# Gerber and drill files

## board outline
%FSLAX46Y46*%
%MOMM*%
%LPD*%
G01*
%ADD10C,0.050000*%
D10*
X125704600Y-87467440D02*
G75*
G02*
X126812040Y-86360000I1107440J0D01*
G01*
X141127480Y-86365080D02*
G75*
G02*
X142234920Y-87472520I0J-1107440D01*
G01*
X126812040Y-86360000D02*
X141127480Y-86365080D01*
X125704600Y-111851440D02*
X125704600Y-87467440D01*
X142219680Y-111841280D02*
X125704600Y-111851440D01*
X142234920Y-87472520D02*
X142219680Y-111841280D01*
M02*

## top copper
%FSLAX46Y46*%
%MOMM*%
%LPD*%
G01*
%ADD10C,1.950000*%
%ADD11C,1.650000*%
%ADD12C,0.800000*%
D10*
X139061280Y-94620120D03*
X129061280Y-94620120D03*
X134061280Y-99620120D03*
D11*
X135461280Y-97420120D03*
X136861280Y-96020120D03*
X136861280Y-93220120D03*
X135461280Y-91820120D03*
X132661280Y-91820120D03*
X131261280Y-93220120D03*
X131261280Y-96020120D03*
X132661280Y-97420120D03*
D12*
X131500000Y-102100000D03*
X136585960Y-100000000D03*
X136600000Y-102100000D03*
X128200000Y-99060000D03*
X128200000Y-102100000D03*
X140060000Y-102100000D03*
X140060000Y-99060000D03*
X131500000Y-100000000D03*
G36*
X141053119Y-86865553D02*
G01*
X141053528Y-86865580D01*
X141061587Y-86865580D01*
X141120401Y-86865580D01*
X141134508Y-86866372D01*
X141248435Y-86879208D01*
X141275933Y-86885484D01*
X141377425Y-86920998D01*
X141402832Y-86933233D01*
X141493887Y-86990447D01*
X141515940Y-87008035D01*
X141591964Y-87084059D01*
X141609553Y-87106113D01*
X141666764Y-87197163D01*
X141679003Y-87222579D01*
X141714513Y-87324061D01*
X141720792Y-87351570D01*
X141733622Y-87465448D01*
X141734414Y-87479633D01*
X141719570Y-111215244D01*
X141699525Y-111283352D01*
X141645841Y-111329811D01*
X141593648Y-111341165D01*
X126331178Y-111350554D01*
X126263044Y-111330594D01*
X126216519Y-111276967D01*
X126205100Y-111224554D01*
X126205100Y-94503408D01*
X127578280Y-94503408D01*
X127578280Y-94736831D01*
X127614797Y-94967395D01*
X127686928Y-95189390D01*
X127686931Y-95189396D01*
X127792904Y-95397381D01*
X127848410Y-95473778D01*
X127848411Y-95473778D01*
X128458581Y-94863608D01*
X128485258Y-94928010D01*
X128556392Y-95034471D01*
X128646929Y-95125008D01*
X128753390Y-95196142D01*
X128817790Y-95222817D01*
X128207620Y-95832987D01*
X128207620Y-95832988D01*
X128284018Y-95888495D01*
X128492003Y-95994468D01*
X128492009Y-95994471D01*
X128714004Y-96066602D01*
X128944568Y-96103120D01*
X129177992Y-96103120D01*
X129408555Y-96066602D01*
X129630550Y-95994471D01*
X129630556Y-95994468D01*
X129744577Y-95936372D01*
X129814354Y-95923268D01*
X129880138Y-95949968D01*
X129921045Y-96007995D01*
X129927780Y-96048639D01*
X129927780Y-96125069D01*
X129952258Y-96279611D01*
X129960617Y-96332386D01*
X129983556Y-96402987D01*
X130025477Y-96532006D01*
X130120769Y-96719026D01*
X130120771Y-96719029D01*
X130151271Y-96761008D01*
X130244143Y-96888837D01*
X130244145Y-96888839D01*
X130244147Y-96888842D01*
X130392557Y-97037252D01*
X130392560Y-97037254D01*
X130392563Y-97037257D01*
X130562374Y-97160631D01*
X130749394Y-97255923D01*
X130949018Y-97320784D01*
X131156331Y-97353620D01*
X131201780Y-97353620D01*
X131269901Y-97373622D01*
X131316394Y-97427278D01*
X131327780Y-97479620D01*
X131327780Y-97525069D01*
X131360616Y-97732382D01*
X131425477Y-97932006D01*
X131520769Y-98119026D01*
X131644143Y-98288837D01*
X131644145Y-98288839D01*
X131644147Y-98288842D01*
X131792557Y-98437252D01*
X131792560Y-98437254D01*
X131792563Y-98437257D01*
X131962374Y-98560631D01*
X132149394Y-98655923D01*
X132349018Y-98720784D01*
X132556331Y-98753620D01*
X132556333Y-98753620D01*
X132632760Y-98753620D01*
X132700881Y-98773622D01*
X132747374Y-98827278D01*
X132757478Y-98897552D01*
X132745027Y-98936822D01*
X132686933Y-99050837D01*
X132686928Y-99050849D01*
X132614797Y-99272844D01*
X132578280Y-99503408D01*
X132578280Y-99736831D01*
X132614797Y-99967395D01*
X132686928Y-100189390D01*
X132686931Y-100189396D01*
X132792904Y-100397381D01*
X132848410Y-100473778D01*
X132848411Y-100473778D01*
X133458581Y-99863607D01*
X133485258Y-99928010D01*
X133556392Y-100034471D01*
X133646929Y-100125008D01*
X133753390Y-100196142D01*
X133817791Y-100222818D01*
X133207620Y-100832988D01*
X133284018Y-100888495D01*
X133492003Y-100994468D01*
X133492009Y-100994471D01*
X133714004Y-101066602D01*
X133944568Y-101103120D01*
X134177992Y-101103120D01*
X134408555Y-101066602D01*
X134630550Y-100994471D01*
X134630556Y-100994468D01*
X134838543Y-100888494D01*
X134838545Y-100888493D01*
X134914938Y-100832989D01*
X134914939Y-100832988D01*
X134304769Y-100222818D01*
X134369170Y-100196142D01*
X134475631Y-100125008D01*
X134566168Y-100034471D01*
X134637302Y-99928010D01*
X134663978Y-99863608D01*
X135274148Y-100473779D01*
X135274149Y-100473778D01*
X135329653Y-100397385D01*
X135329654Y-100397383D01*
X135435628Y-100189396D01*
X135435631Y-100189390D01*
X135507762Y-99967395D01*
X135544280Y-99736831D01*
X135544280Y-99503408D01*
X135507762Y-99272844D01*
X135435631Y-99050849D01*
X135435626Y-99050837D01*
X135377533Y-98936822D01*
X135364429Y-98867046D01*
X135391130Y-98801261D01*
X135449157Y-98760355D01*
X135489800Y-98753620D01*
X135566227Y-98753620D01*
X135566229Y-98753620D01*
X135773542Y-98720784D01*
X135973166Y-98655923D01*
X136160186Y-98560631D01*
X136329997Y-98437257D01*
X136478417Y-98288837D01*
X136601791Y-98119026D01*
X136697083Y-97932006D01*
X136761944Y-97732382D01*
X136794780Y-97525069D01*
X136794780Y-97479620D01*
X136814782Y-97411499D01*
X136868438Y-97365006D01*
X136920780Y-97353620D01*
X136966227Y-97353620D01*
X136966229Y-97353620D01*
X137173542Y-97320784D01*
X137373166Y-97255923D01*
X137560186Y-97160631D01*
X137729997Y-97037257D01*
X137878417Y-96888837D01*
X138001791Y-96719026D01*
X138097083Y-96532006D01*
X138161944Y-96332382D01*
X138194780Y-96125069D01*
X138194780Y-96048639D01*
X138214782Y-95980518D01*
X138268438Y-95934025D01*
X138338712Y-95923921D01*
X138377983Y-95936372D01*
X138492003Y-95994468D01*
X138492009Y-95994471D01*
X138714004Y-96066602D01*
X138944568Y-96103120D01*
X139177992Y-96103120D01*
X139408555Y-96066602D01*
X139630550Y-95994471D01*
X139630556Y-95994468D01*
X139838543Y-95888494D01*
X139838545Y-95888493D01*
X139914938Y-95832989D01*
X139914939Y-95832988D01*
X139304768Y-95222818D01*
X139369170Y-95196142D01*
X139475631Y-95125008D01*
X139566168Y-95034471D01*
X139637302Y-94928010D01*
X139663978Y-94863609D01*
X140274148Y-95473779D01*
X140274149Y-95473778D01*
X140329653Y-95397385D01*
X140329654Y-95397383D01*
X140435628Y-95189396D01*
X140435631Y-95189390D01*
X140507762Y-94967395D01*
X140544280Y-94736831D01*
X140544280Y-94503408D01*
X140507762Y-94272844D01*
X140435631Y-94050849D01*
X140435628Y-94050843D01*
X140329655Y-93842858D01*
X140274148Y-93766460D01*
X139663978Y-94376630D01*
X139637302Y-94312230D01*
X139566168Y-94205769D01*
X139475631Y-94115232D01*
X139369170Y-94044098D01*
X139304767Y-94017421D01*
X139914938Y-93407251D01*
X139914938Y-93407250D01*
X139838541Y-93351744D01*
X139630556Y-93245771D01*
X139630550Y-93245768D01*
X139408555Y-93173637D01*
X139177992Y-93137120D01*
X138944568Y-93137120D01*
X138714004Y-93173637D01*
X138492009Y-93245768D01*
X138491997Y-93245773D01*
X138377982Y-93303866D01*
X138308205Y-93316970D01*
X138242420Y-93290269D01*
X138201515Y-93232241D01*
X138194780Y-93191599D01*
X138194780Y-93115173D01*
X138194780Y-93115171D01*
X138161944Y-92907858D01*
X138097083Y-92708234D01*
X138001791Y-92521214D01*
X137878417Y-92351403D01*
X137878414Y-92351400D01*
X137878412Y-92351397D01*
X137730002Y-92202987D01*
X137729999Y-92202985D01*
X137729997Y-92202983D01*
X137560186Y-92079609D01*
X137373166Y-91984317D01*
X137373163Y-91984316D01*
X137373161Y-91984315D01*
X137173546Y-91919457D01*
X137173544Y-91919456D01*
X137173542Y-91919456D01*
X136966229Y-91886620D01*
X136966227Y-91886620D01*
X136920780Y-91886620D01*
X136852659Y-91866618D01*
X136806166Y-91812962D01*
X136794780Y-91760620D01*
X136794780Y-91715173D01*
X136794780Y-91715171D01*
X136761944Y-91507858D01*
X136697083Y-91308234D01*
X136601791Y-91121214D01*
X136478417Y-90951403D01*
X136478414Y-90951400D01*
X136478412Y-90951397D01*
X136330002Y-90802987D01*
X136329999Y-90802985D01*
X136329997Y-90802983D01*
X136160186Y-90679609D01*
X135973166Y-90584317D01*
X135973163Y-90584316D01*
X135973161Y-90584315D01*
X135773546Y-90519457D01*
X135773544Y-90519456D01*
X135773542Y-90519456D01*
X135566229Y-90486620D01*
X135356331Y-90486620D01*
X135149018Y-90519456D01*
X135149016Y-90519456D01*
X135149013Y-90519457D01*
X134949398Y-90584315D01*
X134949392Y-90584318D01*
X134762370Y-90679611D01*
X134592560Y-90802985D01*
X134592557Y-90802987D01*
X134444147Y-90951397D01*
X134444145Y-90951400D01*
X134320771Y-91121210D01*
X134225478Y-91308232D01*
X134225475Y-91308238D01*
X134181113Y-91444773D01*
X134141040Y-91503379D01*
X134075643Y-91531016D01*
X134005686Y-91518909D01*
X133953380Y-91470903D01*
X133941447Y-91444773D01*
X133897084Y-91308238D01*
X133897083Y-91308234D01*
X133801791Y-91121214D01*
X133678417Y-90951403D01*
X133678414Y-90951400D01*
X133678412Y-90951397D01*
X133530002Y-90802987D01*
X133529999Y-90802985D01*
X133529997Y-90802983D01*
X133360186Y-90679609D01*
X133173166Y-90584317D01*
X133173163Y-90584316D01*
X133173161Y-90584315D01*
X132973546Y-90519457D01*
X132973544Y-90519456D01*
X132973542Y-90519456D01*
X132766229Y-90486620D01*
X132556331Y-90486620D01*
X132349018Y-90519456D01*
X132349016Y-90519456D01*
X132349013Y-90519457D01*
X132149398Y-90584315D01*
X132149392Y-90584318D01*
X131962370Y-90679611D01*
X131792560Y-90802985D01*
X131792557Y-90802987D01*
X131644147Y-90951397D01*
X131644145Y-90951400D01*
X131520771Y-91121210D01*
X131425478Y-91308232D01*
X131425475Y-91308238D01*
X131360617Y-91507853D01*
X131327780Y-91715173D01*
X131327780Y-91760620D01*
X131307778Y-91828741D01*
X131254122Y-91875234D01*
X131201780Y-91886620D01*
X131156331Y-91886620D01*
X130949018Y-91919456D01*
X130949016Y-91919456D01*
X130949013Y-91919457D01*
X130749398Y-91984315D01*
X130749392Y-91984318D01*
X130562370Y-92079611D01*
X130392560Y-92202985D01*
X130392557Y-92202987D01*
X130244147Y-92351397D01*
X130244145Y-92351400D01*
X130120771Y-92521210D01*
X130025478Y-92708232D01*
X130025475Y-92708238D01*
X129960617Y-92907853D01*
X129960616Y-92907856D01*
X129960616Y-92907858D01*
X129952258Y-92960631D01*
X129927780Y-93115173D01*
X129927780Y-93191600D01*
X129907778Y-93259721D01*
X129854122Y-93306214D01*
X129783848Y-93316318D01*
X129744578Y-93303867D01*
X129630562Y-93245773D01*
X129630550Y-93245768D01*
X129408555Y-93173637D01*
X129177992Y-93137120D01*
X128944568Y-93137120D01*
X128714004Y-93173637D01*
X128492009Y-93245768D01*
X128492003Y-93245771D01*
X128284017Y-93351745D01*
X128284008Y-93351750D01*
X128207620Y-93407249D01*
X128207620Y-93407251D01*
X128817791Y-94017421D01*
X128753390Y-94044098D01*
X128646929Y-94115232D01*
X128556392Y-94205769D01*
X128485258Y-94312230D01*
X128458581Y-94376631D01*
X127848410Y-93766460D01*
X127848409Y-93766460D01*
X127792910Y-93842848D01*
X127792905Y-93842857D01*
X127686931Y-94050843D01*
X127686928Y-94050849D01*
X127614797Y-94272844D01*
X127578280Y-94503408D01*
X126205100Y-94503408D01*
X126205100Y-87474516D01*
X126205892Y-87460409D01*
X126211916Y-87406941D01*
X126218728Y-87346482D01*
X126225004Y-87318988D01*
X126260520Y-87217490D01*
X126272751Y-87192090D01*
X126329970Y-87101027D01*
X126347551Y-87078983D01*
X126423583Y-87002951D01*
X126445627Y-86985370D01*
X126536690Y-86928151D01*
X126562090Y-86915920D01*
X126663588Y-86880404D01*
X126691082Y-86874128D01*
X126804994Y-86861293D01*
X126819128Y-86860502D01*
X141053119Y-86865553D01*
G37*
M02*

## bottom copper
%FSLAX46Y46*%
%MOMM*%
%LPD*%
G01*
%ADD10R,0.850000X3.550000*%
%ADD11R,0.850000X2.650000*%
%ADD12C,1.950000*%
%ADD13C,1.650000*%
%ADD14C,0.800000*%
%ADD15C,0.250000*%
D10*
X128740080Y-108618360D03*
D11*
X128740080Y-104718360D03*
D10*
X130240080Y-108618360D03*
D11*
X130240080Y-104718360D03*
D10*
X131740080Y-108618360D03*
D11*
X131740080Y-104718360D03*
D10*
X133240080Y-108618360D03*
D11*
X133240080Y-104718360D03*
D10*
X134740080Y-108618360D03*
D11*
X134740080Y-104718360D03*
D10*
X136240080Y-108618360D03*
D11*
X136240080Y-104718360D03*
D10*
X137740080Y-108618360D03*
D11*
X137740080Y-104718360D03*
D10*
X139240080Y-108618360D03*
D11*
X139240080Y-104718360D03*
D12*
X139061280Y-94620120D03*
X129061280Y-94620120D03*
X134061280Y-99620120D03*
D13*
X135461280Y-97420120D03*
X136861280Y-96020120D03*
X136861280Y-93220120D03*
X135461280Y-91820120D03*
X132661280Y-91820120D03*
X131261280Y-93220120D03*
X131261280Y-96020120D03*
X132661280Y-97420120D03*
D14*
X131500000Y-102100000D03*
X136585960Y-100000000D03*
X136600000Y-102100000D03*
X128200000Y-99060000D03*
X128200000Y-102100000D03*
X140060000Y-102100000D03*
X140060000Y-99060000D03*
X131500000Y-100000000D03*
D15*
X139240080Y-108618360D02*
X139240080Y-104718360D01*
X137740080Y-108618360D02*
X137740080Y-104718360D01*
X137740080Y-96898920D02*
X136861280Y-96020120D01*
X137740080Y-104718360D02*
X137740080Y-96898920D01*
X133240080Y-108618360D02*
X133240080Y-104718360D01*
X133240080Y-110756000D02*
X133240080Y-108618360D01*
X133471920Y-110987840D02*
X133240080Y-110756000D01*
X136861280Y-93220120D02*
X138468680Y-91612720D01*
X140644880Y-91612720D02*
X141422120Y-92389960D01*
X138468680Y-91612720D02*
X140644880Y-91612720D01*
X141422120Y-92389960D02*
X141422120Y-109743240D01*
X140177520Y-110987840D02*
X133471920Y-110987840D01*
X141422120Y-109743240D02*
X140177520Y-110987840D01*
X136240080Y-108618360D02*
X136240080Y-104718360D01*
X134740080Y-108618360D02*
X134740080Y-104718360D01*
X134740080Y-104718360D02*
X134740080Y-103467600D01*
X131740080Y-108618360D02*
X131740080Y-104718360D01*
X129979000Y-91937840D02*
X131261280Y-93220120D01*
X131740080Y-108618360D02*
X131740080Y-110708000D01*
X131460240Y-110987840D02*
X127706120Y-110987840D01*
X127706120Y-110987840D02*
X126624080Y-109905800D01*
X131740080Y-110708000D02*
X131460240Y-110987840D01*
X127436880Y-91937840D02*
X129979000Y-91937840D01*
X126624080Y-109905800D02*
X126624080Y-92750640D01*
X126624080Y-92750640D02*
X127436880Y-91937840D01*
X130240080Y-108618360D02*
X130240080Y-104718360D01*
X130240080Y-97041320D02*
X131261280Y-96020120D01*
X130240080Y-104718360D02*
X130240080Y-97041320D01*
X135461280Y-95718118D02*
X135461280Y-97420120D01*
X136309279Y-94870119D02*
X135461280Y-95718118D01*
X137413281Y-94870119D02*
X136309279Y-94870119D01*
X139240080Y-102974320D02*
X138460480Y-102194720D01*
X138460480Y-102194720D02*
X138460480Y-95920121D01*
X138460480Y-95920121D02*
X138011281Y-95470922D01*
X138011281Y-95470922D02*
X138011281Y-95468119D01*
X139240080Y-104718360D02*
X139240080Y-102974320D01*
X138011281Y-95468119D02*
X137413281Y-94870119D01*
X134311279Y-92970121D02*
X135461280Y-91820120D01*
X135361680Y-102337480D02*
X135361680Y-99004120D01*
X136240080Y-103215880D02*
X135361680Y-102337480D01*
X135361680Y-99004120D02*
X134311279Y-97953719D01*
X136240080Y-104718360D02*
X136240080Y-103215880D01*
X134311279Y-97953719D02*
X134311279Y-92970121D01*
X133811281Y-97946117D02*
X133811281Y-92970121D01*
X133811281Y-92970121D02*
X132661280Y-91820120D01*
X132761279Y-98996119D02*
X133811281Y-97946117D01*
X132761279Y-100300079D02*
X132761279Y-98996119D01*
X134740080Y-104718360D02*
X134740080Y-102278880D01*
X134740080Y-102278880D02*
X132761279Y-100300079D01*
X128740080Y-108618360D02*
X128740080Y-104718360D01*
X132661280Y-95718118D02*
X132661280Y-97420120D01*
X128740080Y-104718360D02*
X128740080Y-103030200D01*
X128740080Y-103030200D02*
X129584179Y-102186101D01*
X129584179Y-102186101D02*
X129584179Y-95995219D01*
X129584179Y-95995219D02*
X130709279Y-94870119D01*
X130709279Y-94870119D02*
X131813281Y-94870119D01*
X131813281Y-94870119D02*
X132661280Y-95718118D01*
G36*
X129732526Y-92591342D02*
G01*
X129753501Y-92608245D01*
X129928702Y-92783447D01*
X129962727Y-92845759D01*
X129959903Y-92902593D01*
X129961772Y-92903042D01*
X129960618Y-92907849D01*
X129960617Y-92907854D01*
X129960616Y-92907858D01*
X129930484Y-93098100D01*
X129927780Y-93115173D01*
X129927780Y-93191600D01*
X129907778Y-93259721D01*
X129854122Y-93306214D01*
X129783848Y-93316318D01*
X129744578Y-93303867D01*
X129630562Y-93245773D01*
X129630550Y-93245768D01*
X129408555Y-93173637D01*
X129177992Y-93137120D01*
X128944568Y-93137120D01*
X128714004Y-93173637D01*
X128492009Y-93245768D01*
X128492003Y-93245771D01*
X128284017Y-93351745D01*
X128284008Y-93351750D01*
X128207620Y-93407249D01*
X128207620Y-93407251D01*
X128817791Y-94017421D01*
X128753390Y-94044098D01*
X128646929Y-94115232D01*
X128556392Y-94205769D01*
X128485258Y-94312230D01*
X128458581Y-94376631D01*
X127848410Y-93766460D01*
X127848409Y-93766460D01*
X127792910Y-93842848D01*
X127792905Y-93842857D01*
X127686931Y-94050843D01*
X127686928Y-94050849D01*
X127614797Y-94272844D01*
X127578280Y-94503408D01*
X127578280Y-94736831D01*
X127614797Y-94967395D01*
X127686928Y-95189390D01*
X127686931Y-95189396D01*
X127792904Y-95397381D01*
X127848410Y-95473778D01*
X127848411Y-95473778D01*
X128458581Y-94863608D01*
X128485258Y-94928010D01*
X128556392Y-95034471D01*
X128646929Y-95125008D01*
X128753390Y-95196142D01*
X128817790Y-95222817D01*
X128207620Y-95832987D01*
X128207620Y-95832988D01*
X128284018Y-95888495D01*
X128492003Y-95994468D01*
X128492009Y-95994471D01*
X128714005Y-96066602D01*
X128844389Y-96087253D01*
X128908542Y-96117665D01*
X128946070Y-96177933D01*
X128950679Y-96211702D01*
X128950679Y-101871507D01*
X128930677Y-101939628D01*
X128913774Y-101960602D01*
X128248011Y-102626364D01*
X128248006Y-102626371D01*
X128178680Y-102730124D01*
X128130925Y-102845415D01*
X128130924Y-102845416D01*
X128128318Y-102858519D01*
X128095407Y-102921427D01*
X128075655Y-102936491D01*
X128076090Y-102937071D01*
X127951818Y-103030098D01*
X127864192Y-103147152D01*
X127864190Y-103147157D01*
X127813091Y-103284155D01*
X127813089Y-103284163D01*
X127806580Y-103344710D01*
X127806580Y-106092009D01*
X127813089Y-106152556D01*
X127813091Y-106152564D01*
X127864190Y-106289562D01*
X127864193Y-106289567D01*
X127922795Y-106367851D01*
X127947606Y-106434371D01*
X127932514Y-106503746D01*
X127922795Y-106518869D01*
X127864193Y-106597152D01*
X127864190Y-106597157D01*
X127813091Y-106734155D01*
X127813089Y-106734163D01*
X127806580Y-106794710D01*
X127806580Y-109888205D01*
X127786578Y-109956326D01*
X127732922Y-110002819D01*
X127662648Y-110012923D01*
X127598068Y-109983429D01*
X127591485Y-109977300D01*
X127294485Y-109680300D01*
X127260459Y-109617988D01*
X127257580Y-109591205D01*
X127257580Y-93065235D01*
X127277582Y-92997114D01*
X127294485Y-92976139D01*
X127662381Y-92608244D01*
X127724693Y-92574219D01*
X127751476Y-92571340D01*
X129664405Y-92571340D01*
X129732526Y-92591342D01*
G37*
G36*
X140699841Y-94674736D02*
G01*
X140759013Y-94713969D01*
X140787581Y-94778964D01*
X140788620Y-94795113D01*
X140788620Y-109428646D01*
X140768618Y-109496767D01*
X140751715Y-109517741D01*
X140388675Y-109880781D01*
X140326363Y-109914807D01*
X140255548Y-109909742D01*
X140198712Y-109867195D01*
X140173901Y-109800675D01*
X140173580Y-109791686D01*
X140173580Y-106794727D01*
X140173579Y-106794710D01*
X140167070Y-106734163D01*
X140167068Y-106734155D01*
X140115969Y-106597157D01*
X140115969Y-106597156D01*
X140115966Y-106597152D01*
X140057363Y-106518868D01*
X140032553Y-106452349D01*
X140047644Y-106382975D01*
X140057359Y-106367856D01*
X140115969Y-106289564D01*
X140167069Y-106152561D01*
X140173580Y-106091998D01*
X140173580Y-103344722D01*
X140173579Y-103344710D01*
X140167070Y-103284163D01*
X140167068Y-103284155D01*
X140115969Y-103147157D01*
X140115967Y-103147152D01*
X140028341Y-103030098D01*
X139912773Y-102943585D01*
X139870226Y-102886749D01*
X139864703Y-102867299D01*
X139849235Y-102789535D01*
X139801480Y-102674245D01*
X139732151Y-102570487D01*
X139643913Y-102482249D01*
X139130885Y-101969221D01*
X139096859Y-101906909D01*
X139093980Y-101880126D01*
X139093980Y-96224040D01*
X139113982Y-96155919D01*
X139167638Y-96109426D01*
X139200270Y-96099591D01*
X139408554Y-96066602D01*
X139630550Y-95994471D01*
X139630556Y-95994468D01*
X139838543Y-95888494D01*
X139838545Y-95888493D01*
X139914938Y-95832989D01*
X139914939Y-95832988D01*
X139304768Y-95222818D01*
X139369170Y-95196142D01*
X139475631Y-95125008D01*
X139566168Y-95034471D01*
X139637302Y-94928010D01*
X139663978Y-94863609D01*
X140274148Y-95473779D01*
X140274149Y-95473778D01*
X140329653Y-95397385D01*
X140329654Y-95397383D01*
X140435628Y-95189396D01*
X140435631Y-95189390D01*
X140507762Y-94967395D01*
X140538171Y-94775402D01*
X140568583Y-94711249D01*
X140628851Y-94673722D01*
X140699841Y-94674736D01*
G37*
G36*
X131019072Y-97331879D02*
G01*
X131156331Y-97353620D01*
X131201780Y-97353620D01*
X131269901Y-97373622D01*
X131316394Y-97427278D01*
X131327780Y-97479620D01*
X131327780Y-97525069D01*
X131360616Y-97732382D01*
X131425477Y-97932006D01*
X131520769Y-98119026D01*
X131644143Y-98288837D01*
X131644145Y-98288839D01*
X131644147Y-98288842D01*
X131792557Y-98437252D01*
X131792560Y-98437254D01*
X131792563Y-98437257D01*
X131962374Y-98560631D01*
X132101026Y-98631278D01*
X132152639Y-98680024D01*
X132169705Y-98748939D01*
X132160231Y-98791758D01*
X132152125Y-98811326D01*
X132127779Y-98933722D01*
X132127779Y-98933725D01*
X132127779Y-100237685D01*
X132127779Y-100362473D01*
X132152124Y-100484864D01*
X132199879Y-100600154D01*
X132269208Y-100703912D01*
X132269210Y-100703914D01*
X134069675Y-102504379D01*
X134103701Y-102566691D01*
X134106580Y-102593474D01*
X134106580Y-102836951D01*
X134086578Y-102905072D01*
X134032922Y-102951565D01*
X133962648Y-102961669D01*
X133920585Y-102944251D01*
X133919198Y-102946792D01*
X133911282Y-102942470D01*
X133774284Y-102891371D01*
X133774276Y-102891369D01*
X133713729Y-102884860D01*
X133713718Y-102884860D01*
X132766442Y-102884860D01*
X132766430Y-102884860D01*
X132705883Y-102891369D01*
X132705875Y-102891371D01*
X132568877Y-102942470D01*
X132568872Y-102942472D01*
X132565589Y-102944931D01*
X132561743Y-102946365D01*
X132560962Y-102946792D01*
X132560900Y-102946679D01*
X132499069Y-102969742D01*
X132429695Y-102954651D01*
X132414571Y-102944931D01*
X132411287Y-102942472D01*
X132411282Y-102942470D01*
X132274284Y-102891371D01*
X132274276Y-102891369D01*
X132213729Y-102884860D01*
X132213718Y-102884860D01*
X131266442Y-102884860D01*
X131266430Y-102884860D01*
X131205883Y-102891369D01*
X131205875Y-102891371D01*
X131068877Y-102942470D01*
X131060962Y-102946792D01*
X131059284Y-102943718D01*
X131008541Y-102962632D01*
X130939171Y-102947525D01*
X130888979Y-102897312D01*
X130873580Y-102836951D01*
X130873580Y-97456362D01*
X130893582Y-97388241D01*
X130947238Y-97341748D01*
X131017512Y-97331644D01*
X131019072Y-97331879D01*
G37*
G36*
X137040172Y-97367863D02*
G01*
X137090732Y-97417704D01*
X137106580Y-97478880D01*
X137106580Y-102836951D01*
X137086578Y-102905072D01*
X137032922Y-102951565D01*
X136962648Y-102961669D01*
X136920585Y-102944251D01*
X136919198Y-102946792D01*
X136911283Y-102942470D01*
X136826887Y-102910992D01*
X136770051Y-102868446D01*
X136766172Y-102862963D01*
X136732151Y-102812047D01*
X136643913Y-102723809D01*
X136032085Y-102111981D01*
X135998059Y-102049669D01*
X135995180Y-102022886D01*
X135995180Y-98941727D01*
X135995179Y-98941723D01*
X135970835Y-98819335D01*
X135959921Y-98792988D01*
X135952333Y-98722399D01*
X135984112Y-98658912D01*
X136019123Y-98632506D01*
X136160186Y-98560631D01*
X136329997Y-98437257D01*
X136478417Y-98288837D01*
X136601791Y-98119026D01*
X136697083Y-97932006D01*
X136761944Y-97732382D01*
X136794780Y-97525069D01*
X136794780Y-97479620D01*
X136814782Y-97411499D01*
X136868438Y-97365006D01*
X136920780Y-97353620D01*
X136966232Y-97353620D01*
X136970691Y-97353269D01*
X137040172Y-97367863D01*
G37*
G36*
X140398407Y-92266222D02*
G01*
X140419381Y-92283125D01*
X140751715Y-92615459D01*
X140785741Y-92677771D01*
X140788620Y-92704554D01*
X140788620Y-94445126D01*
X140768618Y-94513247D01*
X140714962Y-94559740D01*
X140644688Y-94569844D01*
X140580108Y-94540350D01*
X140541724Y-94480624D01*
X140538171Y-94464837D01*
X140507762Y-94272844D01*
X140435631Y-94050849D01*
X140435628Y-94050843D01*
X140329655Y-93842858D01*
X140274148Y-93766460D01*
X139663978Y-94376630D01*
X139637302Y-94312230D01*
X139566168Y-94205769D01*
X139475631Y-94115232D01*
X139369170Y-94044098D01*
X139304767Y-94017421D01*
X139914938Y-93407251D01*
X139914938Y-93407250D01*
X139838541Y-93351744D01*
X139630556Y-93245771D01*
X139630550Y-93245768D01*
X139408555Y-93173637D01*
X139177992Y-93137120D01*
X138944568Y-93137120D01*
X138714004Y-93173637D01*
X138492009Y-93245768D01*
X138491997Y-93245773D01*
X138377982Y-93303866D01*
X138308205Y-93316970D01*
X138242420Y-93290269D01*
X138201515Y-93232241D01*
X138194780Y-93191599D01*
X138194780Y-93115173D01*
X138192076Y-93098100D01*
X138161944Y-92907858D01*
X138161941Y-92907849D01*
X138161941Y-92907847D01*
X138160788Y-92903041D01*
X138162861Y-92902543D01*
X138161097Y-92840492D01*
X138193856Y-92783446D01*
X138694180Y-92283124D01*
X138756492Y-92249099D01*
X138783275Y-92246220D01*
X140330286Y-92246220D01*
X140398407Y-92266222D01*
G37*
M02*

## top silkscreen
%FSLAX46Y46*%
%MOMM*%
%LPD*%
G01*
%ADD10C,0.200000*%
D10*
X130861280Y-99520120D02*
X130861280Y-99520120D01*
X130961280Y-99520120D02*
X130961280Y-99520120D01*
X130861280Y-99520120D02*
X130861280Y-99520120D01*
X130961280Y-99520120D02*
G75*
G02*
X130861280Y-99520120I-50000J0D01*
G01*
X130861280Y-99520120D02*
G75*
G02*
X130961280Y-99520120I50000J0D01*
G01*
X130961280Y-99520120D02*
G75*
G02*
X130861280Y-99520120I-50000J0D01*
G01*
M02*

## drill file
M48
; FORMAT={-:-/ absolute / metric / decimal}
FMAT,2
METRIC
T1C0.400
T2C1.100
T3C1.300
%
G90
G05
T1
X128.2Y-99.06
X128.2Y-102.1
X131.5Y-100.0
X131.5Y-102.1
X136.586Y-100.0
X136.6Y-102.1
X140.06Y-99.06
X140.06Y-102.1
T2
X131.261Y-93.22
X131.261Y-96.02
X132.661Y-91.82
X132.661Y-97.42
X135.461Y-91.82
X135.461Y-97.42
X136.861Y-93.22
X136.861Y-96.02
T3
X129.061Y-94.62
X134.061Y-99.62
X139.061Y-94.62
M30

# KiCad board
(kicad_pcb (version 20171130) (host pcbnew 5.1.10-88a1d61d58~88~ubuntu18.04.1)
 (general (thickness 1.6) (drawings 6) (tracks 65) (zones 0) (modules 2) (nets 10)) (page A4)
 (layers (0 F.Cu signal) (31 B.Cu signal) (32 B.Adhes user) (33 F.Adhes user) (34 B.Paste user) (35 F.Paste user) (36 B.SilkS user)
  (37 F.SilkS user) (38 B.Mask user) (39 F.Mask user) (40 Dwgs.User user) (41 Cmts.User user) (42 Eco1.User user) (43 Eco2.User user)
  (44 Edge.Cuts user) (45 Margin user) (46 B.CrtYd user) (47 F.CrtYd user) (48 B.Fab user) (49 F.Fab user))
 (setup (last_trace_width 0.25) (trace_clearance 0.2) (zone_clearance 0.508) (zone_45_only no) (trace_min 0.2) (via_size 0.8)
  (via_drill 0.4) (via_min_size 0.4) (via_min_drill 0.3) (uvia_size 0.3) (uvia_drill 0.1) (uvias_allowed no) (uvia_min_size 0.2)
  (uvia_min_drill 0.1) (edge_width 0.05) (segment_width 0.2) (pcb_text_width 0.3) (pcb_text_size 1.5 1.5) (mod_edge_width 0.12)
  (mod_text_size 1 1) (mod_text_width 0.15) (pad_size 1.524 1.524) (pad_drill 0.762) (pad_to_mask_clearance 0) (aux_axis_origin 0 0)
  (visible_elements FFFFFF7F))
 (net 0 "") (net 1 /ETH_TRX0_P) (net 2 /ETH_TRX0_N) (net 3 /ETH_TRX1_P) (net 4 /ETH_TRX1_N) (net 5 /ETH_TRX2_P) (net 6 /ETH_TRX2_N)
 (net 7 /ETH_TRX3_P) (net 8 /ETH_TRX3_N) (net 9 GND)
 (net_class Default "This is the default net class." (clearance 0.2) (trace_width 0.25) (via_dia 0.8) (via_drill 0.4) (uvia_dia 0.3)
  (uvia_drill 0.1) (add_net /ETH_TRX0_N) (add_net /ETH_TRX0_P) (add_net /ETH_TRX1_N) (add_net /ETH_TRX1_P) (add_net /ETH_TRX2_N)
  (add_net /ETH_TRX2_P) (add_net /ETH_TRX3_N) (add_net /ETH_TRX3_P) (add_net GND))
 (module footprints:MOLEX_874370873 (layer B.Cu) (at 133.99008 106.89336 180)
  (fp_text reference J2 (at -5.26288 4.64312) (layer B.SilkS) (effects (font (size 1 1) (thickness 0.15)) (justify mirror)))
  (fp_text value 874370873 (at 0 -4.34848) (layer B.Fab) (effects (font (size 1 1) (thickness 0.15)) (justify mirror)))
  (pad 8_2 smd rect (at 5.25 -1.725 180) (size 0.85 3.55) (layers B.Cu B.Paste) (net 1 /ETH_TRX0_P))
  (pad 8_1 smd rect (at 5.25 2.175 180) (size 0.85 2.65) (layers B.Cu B.Paste) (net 1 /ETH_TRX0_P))
  (pad 7_2 smd rect (at 3.75 -1.725 180) (size 0.85 3.55) (layers B.Cu B.Paste) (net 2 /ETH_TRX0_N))
  (pad 7_1 smd rect (at 3.75 2.175 180) (size 0.85 2.65) (layers B.Cu B.Paste) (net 2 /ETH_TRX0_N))
  (pad 6_2 smd rect (at 2.25 -1.725 180) (size 0.85 3.55) (layers B.Cu B.Paste) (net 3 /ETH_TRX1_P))
  (pad 6_1 smd rect (at 2.25 2.175 180) (size 0.85 2.65) (layers B.Cu B.Paste) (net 3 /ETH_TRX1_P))
  (pad 5_2 smd rect (at 0.75 -1.725 180) (size 0.85 3.55) (layers B.Cu B.Paste) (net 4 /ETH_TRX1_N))
  (pad 5_1 smd rect (at 0.75 2.175 180) (size 0.85 2.65) (layers B.Cu B.Paste) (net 4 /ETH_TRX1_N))
  (pad 4_2 smd rect (at -0.75 -1.725 180) (size 0.85 3.55) (layers B.Cu B.Paste) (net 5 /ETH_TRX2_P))
  (pad 4_1 smd rect (at -0.75 2.175 180) (size 0.85 2.65) (layers B.Cu B.Paste) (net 5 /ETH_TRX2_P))
  (pad 3_2 smd rect (at -2.25 -1.725 180) (size 0.85 3.55) (layers B.Cu B.Paste) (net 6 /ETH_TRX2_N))
  (pad 3_1 smd rect (at -2.25 2.175 180) (size 0.85 2.65) (layers B.Cu B.Paste) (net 6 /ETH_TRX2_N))
  (pad 2_2 smd rect (at -3.75 -1.725 180) (size 0.85 3.55) (layers B.Cu B.Paste) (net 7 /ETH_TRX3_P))
  (pad 2_1 smd rect (at -3.75 2.175 180) (size 0.85 2.65) (layers B.Cu B.Paste) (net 7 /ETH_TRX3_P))
  (pad 1_2 smd rect (at -5.25 -1.725 180) (size 0.85 3.55) (layers B.Cu B.Paste) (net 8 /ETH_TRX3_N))
  (pad 1_1 smd rect (at -5.25 2.175 180) (size 0.85 2.65) (layers B.Cu B.Paste) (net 8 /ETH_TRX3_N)))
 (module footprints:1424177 (layer F.Cu) (at 132.16128 100.02012)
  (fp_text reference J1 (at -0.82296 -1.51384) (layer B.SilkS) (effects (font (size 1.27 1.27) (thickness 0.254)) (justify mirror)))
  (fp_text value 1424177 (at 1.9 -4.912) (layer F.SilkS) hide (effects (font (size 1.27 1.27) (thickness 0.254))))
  (fp_line (start -1.3 -0.5) (end -1.3 -0.5) (layer F.SilkS) (width 0.2))
  (fp_line (start -1.2 -0.5) (end -1.2 -0.5) (layer F.SilkS) (width 0.2))
  (fp_line (start -1.3 -0.5) (end -1.3 -0.5) (layer F.SilkS) (width 0.2))
  (fp_arc (start -1.25 -0.5) (end -1.3 -0.5) (angle -180) (layer F.SilkS) (width 0.2))
  (fp_arc (start -1.25 -0.5) (end -1.2 -0.5) (angle -180) (layer F.SilkS) (width 0.2))
  (fp_arc (start -1.25 -0.5) (end -1.3 -0.5) (angle -180) (layer F.SilkS) (width 0.2))
  (pad MH3 thru_hole circle (at 6.9 -5.4) (size 1.95 1.95) (drill 1.3) (layers *.Cu *.Mask) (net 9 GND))
  (pad MH2 thru_hole circle (at -3.1 -5.4) (size 1.95 1.95) (drill 1.3) (layers *.Cu *.Mask) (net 9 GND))
  (pad MH1 thru_hole circle (at 1.9 -0.4) (size 1.95 1.95) (drill 1.3) (layers *.Cu *.Mask) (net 9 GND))
  (pad 8 thru_hole circle (at 3.3 -2.6) (size 1.65 1.65) (drill 1.1) (layers *.Cu *.Mask) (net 8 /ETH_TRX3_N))
  (pad 7 thru_hole circle (at 4.7 -4) (size 1.65 1.65) (drill 1.1) (layers *.Cu *.Mask) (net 7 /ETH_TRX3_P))
  (pad 6 thru_hole circle (at 4.7 -6.8) (size 1.65 1.65) (drill 1.1) (layers *.Cu *.Mask) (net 4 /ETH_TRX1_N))
  (pad 5 thru_hole circle (at 3.3 -8.2) (size 1.65 1.65) (drill 1.1) (layers *.Cu *.Mask) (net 6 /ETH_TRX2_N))
  (pad 4 thru_hole circle (at 0.5 -8.2) (size 1.65 1.65) (drill 1.1) (layers *.Cu *.Mask) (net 5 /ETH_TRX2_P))
  (pad 3 thru_hole circle (at -0.9 -6.8) (size 1.65 1.65) (drill 1.1) (layers *.Cu *.Mask) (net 3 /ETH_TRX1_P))
  (pad 2 thru_hole circle (at -0.9 -4) (size 1.65 1.65) (drill 1.1) (layers *.Cu *.Mask) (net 2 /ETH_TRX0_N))
  (pad 1 thru_hole circle (at 0.5 -2.6) (size 1.65 1.65) (drill 1.1) (layers *.Cu *.Mask) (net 1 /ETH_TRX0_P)))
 (gr_arc (start 126.81204 87.46744) (end 126.81204 86.36) (angle -90) (layer Edge.Cuts) (width 0.05))
 (gr_arc (start 141.12748 87.47252) (end 142.23492 87.47252) (angle -90) (layer Edge.Cuts) (width 0.05))
 (gr_line (start 126.81204 86.36) (end 141.12748 86.36508) (layer Edge.Cuts) (width 0.05))
 (gr_line (start 125.7046 111.85144) (end 125.7046 87.46744) (layer Edge.Cuts) (width 0.05))
 (gr_line (start 142.21968 111.84128) (end 125.7046 111.85144) (layer Edge.Cuts) (width 0.05))
 (gr_line (start 142.23492 87.47252) (end 142.21968 111.84128) (layer Edge.Cuts) (width 0.05))
 (via (at 131.5 102.1) (size 0.8) (drill 0.4) (layers F.Cu B.Cu) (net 9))
 (via (at 136.58596 100) (size 0.8) (drill 0.4) (layers F.Cu B.Cu) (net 9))
 (via (at 136.6 102.1) (size 0.8) (drill 0.4) (layers F.Cu B.Cu) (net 9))
 (via (at 128.2 99.06) (size 0.8) (drill 0.4) (layers F.Cu B.Cu) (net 9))
 (via (at 128.2 102.1) (size 0.8) (drill 0.4) (layers F.Cu B.Cu) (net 9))
 (via (at 140.06 102.1) (size 0.8) (drill 0.4) (layers F.Cu B.Cu) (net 9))
 (via (at 140.06 99.06) (size 0.8) (drill 0.4) (layers F.Cu B.Cu) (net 9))
 (segment (start 139.24008 108.61836) (end 139.24008 104.71836) (width 0.25) (layer B.Cu) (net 8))
 (segment (start 137.74008 108.61836) (end 137.74008 104.71836) (width 0.25) (layer B.Cu) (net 7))
 (segment (start 137.74008 96.89892) (end 136.86128 96.02012) (width 0.25) (layer B.Cu) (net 7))
 (segment (start 137.74008 104.71836) (end 137.74008 96.89892) (width 0.25) (layer B.Cu) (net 7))
 (segment (start 133.24008 108.61836) (end 133.24008 104.71836) (width 0.25) (layer B.Cu) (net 4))
 (segment (start 133.24008 110.756) (end 133.24008 108.61836) (width 0.25) (layer B.Cu) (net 4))
 (segment (start 133.47192 110.98784) (end 133.24008 110.756) (width 0.25) (layer B.Cu) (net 4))
 (segment (start 136.86128 93.22012) (end 138.46868 91.61272) (width 0.25) (layer B.Cu) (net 4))
 (segment (start 140.64488 91.61272) (end 141.42212 92.38996) (width 0.25) (layer B.Cu) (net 4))
 (segment (start 138.46868 91.61272) (end 140.64488 91.61272) (width 0.25) (layer B.Cu) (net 4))
 (segment (start 141.42212 92.38996) (end 141.42212 109.74324) (width 0.25) (layer B.Cu) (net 4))
 (segment (start 140.17752 110.98784) (end 133.47192 110.98784) (width 0.25) (layer B.Cu) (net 4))
 (segment (start 141.42212 109.74324) (end 140.17752 110.98784) (width 0.25) (layer B.Cu) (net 4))
 (segment (start 136.24008 108.61836) (end 136.24008 104.71836) (width 0.25) (layer B.Cu) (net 6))
 (segment (start 134.74008 108.61836) (end 134.74008 104.71836) (width 0.25) (layer B.Cu) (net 5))
 (segment (start 134.74008 104.71836) (end 134.74008 103.4676) (width 0.25) (layer B.Cu) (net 5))
 (segment (start 131.74008 108.61836) (end 131.74008 104.71836) (width 0.25) (layer B.Cu) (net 3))
 (segment (start 129.979 91.93784) (end 131.26128 93.22012) (width 0.25) (layer B.Cu) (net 3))
 (segment (start 131.74008 108.61836) (end 131.74008 110.708) (width 0.25) (layer B.Cu) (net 3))
 (segment (start 131.46024 110.98784) (end 127.70612 110.98784) (width 0.25) (layer B.Cu) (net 3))
 (segment (start 127.70612 110.98784) (end 126.62408 109.9058) (width 0.25) (layer B.Cu) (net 3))
 (segment (start 131.74008 110.708) (end 131.46024 110.98784) (width 0.25) (layer B.Cu) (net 3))
 (segment (start 127.43688 91.93784) (end 129.979 91.93784) (width 0.25) (layer B.Cu) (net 3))
 (segment (start 126.62408 109.9058) (end 126.62408 92.75064) (width 0.25) (layer B.Cu) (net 3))
 (segment (start 126.62408 92.75064) (end 127.43688 91.93784) (width 0.25) (layer B.Cu) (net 3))
 (segment (start 130.24008 108.61836) (end 130.24008 104.71836) (width 0.25) (layer B.Cu) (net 2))
 (segment (start 130.24008 97.04132) (end 131.26128 96.02012) (width 0.25) (layer B.Cu) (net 2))
 (segment (start 130.24008 104.71836) (end 130.24008 97.04132) (width 0.25) (layer B.Cu) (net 2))
 (via (at 131.5 100) (size 0.8) (drill 0.4) (layers F.Cu B.Cu) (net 9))
 (segment (start 135.46128 95.718118) (end 135.46128 97.42012) (width 0.25) (layer B.Cu) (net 8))
 (segment (start 136.309279 94.870119) (end 135.46128 95.718118) (width 0.25) (layer B.Cu) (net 8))
 (segment (start 137.413281 94.870119) (end 136.309279 94.870119) (width 0.25) (layer B.Cu) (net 8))
 (segment (start 139.24008 102.97432) (end 138.46048 102.19472) (width 0.25) (layer B.Cu) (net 8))
 (segment (start 138.46048 102.19472) (end 138.46048 95.920121) (width 0.25) (layer B.Cu) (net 8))
 (segment (start 138.46048 95.920121) (end 138.011281 95.470922) (width 0.25) (layer B.Cu) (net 8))
 (segment (start 138.011281 95.470922) (end 138.011281 95.468119) (width 0.25) (layer B.Cu) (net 8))
 (segment (start 139.24008 104.71836) (end 139.24008 102.97432) (width 0.25) (layer B.Cu) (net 8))
 (segment (start 138.011281 95.468119) (end 137.413281 94.870119) (width 0.25) (layer B.Cu) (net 8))
 (segment (start 134.311279 92.970121) (end 135.46128 91.82012) (width 0.25) (layer B.Cu) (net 6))
 (segment (start 135.36168 102.33748) (end 135.36168 99.00412) (width 0.25) (layer B.Cu) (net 6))
 (segment (start 136.24008 103.21588) (end 135.36168 102.33748) (width 0.25) (layer B.Cu) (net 6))
 (segment (start 135.36168 99.00412) (end 134.311279 97.953719) (width 0.25) (layer B.Cu) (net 6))
 (segment (start 136.24008 104.71836) (end 136.24008 103.21588) (width 0.25) (layer B.Cu) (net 6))
 (segment (start 134.311279 97.953719) (end 134.311279 92.970121) (width 0.25) (layer B.Cu) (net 6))
 (segment (start 133.811281 97.946117) (end 133.811281 92.970121) (width 0.25) (layer B.Cu) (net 5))
 (segment (start 133.811281 92.970121) (end 132.66128 91.82012) (width 0.25) (layer B.Cu) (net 5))
 (segment (start 132.761279 98.996119) (end 133.811281 97.946117) (width 0.25) (layer B.Cu) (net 5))
 (segment (start 132.761279 100.300079) (end 132.761279 98.996119) (width 0.25) (layer B.Cu) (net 5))
 (segment (start 134.74008 104.71836) (end 134.74008 102.27888) (width 0.25) (layer B.Cu) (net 5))
 (segment (start 134.74008 102.27888) (end 132.761279 100.300079) (width 0.25) (layer B.Cu) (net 5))
 (segment (start 128.74008 108.61836) (end 128.74008 104.71836) (width 0.25) (layer B.Cu) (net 1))
 (segment (start 132.66128 95.718118) (end 132.66128 97.42012) (width 0.25) (layer B.Cu) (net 1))
 (segment (start 128.74008 104.71836) (end 128.74008 103.0302) (width 0.25) (layer B.Cu) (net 1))
 (segment (start 128.74008 103.0302) (end 129.584179 102.186101) (width 0.25) (layer B.Cu) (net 1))
 (segment (start 129.584179 102.186101) (end 129.584179 95.995219) (width 0.25) (layer B.Cu) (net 1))
 (segment (start 129.584179 95.995219) (end 130.709279 94.870119) (width 0.25) (layer B.Cu) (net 1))
 (segment (start 130.709279 94.870119) (end 131.813281 94.870119) (width 0.25) (layer B.Cu) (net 1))
 (segment (start 131.813281 94.870119) (end 132.66128 95.718118) (width 0.25) (layer B.Cu) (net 1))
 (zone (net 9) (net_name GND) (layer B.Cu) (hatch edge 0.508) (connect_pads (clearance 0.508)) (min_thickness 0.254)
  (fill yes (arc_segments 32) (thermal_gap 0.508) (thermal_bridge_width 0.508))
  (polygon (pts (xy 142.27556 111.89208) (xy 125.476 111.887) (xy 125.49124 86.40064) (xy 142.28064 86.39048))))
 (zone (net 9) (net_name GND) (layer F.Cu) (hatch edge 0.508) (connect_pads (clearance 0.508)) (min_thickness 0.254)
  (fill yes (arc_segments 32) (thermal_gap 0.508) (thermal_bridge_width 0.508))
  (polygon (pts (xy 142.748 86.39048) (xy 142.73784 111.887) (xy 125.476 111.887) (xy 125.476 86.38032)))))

